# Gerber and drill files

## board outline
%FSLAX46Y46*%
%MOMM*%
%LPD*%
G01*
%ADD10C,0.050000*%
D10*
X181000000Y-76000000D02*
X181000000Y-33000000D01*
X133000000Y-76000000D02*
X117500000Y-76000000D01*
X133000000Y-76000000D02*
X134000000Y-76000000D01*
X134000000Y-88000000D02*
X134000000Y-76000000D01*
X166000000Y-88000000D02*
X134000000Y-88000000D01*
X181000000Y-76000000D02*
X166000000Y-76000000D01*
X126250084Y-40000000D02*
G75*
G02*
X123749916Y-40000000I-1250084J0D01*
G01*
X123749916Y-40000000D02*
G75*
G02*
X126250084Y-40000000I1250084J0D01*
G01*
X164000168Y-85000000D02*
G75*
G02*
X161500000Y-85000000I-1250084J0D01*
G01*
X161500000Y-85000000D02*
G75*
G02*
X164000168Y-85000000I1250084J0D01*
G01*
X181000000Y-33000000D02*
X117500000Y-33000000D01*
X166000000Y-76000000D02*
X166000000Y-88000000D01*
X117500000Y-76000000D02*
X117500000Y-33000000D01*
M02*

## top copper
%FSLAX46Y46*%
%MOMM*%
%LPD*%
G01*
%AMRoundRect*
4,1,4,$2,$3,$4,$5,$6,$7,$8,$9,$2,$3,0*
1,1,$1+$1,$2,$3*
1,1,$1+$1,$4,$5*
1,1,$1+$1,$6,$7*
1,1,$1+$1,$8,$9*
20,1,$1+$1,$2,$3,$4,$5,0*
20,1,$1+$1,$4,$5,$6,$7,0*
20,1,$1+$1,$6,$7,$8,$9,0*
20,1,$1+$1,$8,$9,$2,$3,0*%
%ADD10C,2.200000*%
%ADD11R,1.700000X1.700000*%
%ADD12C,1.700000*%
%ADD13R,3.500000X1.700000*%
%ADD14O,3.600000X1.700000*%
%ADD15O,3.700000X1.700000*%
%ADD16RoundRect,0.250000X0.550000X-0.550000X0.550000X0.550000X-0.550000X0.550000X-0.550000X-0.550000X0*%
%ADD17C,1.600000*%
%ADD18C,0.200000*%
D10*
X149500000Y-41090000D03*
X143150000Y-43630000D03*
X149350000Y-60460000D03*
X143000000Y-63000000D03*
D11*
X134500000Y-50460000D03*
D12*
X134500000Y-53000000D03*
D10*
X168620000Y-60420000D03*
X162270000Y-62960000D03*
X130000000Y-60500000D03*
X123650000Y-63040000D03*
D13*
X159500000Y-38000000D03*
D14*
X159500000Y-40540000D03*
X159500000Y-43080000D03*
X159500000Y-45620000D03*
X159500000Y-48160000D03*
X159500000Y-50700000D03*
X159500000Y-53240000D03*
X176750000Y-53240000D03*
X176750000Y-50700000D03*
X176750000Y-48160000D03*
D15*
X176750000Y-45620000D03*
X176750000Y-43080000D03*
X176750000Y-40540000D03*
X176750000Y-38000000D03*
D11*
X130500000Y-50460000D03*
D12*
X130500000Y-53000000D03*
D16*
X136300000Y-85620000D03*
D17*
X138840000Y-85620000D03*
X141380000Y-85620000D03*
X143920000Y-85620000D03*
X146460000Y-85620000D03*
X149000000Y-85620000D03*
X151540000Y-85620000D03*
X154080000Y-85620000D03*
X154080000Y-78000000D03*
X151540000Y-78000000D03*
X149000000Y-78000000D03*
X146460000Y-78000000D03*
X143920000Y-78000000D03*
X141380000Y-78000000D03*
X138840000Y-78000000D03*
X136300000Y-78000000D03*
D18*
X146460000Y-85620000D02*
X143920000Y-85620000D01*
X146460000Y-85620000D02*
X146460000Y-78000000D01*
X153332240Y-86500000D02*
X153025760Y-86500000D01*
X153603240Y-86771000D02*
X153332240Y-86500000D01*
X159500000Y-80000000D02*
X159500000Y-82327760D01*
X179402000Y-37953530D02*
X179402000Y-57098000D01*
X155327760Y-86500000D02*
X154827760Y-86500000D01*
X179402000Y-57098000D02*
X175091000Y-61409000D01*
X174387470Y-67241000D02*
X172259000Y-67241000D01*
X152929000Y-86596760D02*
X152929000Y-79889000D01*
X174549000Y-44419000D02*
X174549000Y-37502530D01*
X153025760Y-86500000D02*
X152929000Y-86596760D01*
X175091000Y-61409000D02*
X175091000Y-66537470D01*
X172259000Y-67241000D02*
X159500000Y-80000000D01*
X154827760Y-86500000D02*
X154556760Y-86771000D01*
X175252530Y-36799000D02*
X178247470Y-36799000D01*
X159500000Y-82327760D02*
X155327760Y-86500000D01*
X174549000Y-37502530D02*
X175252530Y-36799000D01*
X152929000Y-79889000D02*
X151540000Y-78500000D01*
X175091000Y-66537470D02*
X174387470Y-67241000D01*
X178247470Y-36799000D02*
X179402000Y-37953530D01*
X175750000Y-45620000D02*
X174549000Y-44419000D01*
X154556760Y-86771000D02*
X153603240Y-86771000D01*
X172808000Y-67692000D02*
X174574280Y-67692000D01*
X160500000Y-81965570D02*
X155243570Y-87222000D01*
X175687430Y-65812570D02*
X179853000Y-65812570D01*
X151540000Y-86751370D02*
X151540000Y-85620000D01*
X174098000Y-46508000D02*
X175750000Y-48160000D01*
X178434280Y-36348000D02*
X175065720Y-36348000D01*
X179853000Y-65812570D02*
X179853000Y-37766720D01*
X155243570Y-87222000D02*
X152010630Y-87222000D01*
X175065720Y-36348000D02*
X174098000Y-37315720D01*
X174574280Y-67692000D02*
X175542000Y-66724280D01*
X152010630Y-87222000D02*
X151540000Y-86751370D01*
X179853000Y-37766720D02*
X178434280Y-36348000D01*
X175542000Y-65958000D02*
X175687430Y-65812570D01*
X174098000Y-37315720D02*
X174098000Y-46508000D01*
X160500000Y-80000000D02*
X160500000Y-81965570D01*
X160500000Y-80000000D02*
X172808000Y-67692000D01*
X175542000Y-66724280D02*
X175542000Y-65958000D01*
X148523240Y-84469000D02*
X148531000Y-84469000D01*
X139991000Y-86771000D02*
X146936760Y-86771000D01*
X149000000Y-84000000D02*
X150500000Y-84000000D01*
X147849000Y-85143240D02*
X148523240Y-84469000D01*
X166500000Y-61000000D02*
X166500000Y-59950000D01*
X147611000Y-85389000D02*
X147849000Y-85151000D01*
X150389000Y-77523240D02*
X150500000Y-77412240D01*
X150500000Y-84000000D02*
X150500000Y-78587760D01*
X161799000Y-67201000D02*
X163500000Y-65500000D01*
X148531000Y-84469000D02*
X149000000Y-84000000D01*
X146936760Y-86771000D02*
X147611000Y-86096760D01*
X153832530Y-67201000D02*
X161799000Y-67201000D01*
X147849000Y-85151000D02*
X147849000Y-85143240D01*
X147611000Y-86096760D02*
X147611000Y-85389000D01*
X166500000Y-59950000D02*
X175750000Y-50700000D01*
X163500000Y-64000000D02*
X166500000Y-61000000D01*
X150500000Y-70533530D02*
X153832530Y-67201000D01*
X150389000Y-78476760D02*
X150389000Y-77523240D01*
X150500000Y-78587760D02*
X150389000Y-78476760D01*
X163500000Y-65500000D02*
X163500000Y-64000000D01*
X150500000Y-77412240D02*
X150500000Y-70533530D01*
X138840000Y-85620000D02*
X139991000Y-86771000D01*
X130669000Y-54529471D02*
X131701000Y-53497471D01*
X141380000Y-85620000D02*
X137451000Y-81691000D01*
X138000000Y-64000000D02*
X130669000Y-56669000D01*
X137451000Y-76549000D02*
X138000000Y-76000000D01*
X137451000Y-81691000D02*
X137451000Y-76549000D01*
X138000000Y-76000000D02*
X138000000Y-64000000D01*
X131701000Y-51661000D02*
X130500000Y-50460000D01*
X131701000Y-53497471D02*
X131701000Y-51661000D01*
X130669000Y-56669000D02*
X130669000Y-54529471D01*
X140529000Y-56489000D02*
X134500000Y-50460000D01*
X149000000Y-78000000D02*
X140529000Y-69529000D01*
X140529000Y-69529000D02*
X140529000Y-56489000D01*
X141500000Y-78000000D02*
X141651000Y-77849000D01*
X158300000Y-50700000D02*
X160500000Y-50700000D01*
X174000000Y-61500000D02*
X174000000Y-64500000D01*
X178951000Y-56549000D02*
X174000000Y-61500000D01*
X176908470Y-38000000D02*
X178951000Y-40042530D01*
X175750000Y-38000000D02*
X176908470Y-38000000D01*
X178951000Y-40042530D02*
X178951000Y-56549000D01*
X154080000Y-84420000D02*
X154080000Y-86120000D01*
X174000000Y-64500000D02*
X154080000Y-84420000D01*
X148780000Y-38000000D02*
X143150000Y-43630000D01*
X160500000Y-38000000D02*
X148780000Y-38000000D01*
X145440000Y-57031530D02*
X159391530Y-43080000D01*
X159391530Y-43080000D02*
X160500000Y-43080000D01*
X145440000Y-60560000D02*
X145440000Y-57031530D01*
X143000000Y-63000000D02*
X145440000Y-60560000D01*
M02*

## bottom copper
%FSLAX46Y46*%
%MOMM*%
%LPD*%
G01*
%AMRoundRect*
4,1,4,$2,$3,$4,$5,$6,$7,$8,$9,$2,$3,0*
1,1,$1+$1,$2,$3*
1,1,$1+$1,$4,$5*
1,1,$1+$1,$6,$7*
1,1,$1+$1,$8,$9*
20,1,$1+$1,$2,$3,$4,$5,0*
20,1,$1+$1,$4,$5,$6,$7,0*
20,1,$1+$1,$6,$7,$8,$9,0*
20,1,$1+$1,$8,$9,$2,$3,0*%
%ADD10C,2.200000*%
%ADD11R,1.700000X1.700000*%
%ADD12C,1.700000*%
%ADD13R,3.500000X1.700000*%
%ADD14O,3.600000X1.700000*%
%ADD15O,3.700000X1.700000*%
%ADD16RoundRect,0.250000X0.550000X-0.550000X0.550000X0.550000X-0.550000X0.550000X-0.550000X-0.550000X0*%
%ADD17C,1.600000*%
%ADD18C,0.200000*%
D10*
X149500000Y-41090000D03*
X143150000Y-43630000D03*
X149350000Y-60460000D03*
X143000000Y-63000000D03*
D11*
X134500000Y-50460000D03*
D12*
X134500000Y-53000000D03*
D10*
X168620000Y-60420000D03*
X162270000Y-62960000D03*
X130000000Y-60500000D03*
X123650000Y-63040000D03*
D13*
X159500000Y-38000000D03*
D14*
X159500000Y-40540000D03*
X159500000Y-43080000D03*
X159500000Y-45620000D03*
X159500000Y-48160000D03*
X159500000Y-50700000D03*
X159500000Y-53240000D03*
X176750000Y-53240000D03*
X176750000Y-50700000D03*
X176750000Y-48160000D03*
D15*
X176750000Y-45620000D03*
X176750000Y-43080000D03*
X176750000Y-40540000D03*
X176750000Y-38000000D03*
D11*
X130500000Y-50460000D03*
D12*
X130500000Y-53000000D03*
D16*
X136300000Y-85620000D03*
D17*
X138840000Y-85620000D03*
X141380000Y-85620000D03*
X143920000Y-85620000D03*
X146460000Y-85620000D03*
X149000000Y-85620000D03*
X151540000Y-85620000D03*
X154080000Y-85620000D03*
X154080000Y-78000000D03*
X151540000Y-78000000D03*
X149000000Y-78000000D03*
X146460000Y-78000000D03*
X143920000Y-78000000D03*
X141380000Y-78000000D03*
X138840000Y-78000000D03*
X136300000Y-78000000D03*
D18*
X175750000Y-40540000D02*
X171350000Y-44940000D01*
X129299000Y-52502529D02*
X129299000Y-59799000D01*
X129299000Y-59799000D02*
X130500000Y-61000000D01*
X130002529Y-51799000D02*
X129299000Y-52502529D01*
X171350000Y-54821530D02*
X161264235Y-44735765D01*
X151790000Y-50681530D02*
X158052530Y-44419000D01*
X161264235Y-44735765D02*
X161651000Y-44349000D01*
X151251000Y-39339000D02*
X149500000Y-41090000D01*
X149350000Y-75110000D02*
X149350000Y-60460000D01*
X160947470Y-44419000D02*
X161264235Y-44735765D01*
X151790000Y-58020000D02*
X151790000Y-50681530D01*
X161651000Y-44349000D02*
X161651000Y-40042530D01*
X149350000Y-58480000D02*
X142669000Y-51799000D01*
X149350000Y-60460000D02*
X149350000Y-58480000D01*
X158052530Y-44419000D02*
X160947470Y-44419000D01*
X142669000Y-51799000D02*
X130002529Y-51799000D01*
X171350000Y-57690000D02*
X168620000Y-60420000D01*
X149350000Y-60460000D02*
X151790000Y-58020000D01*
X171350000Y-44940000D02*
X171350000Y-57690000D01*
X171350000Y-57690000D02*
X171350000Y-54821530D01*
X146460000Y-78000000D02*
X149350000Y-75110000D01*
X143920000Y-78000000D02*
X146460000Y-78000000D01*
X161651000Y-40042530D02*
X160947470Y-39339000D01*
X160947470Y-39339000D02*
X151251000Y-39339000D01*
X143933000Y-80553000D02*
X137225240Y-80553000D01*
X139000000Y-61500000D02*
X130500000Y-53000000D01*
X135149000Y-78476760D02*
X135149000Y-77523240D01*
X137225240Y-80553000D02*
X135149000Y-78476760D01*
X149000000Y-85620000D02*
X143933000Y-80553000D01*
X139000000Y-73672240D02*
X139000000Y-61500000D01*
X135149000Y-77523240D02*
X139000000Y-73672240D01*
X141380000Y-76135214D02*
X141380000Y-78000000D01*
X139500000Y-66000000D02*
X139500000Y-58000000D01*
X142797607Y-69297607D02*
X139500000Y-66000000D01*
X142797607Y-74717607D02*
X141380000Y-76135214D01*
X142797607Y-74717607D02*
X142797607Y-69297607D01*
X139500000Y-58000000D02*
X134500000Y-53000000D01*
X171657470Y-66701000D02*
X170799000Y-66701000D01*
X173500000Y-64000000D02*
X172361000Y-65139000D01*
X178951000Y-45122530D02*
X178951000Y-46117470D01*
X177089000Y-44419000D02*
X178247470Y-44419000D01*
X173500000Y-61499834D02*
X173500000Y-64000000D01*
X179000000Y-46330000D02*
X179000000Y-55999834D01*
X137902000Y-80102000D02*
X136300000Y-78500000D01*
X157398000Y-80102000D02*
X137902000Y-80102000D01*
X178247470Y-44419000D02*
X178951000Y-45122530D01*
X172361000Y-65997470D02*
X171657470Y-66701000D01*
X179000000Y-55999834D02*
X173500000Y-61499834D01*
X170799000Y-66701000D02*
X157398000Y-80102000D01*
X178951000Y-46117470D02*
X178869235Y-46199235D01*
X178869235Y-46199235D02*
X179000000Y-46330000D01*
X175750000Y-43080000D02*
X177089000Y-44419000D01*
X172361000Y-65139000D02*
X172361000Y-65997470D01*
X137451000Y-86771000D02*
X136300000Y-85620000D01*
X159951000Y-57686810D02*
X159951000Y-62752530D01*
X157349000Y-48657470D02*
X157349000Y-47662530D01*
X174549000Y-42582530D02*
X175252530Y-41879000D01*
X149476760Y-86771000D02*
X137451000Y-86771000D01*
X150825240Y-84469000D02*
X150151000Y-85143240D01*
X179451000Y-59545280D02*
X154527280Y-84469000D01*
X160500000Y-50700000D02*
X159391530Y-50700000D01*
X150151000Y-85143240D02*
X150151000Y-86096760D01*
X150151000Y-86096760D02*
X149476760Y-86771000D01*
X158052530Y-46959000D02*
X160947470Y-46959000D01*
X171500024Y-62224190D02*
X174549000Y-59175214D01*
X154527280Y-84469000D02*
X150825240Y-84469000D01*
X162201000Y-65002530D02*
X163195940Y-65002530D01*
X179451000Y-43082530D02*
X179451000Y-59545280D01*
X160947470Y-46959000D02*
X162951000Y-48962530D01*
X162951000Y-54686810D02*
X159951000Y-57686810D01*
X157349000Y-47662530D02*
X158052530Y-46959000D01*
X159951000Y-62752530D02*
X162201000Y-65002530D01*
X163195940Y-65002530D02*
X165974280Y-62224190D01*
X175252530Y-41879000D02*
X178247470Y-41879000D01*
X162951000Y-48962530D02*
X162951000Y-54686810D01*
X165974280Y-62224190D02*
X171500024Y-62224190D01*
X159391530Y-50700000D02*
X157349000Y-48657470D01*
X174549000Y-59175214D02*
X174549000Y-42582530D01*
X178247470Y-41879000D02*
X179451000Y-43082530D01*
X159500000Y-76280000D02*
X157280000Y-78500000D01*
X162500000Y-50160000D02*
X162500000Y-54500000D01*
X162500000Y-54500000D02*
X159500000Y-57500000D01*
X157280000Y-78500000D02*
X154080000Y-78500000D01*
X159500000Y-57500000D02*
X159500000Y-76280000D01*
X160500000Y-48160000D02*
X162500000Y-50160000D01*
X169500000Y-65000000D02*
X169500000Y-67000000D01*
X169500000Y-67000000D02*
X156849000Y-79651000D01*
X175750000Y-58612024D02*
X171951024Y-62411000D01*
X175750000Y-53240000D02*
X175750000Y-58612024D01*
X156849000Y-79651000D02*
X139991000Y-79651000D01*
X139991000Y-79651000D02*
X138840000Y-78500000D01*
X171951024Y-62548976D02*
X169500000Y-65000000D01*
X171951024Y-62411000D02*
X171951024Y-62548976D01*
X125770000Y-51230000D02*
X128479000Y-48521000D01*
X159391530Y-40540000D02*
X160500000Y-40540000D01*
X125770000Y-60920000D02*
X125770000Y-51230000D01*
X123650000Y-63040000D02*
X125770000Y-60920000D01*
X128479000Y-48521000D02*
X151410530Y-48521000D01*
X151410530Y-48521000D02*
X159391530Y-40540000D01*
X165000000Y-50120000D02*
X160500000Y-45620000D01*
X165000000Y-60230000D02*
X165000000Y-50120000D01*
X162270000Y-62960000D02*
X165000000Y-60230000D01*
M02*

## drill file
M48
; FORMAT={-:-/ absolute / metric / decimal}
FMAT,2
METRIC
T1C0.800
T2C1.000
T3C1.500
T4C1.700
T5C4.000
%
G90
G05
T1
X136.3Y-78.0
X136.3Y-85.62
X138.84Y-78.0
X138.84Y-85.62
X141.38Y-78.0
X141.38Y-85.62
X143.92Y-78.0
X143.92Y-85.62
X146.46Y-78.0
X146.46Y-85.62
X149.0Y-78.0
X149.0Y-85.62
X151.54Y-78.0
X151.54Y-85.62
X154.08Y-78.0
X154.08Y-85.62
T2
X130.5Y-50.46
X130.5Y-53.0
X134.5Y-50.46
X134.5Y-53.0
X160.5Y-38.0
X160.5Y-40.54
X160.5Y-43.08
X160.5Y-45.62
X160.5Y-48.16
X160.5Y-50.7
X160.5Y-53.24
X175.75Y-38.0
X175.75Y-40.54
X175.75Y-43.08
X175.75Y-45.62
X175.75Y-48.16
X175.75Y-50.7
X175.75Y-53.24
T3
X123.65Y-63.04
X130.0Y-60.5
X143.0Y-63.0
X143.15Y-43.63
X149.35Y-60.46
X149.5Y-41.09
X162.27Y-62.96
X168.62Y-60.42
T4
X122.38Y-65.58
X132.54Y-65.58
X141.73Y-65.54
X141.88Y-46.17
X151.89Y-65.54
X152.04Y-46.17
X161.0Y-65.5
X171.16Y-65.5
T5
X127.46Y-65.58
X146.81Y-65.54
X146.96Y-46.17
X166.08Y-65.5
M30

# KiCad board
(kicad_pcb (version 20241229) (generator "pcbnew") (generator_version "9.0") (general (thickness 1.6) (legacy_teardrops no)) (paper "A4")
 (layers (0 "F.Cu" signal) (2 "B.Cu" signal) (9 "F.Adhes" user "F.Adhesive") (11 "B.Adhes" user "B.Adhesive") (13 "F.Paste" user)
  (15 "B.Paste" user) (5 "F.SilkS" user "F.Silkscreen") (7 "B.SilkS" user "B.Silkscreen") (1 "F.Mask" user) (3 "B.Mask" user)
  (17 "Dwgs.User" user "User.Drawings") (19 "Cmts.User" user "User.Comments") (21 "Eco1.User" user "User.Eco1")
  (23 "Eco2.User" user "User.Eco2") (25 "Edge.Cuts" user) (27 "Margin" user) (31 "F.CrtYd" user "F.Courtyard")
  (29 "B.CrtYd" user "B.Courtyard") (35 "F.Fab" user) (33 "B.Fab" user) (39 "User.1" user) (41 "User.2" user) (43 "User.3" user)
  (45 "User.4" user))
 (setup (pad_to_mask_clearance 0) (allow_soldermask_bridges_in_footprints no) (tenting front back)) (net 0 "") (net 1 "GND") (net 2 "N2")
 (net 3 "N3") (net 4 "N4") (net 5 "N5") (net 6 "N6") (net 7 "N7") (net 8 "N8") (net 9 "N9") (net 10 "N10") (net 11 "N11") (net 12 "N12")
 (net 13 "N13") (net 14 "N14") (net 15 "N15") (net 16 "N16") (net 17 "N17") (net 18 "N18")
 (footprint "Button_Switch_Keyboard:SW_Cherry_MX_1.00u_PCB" (layer "F.Cu") (at 149.5 41.09)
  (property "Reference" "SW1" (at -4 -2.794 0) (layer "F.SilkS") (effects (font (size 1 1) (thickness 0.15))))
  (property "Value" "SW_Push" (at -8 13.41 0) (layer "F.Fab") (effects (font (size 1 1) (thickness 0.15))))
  (pad "" np_thru_hole circle (at -7.62 5.08) (size 1.7 1.7) (drill 1.7) (layers "*.Cu" "*.Mask"))
  (pad "" np_thru_hole circle (at -2.54 5.08) (size 4 4) (drill 4) (layers "*.Cu" "*.Mask"))
  (pad "" np_thru_hole circle (at 2.54 5.08) (size 1.7 1.7) (drill 1.7) (layers "*.Cu" "*.Mask"))
  (pad "1" thru_hole circle (at 0 0) (size 2.2 2.2) (drill 1.5) (layers "*.Cu" "*.Mask") (remove_unused_layers no) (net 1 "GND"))
  (pad "2" thru_hole circle (at -6.35 2.54) (size 2.2 2.2) (drill 1.5) (layers "*.Cu" "*.Mask") (remove_unused_layers no) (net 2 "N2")))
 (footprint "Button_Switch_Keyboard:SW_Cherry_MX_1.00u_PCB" (layer "F.Cu") (at 149.35 60.46)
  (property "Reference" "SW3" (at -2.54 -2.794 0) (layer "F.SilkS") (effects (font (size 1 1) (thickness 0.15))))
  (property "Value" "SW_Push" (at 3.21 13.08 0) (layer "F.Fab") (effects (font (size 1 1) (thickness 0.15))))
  (pad "" np_thru_hole circle (at -7.62 5.08) (size 1.7 1.7) (drill 1.7) (layers "*.Cu" "*.Mask"))
  (pad "" np_thru_hole circle (at -2.54 5.08) (size 4 4) (drill 4) (layers "*.Cu" "*.Mask"))
  (pad "" np_thru_hole circle (at 2.54 5.08) (size 1.7 1.7) (drill 1.7) (layers "*.Cu" "*.Mask"))
  (pad "1" thru_hole circle (at 0 0) (size 2.2 2.2) (drill 1.5) (layers "*.Cu" "*.Mask") (remove_unused_layers no) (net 1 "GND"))
  (pad "2" thru_hole circle (at -6.35 2.54) (size 2.2 2.2) (drill 1.5) (layers "*.Cu" "*.Mask") (remove_unused_layers no) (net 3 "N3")))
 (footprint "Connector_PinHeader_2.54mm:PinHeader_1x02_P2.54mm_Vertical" (layer "F.Cu") (at 134.5 50.46)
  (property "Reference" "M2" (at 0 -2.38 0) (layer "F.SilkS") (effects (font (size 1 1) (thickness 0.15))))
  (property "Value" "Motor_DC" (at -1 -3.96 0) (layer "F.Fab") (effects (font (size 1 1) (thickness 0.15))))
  (pad "1" thru_hole rect (at 0 0) (size 1.7 1.7) (drill 1) (layers "*.Cu" "*.Mask") (remove_unused_layers no) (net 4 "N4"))
  (pad "2" thru_hole circle (at 0 2.54) (size 1.7 1.7) (drill 1) (layers "*.Cu" "*.Mask") (remove_unused_layers no) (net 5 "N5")))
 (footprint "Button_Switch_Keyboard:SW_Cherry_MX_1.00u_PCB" (layer "F.Cu") (at 168.62 60.42)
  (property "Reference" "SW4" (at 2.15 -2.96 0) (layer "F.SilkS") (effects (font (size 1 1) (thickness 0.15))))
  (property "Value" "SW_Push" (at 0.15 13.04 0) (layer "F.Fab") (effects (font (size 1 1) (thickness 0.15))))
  (pad "" np_thru_hole circle (at -7.62 5.08) (size 1.7 1.7) (drill 1.7) (layers "*.Cu" "*.Mask"))
  (pad "" np_thru_hole circle (at -2.54 5.08) (size 4 4) (drill 4) (layers "*.Cu" "*.Mask"))
  (pad "" np_thru_hole circle (at 2.54 5.08) (size 1.7 1.7) (drill 1.7) (layers "*.Cu" "*.Mask"))
  (pad "1" thru_hole circle (at 0 0) (size 2.2 2.2) (drill 1.5) (layers "*.Cu" "*.Mask") (remove_unused_layers no) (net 1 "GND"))
  (pad "2" thru_hole circle (at -6.35 2.54) (size 2.2 2.2) (drill 1.5) (layers "*.Cu" "*.Mask") (remove_unused_layers no) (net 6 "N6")))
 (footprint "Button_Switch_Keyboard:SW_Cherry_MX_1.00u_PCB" (layer "F.Cu") (at 130 60.5)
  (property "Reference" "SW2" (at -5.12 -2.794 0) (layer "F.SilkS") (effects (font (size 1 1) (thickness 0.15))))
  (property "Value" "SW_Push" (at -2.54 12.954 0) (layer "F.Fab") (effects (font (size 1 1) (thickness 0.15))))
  (pad "" np_thru_hole circle (at -7.62 5.08) (size 1.7 1.7) (drill 1.7) (layers "*.Cu" "*.Mask"))
  (pad "" np_thru_hole circle (at -2.54 5.08) (size 4 4) (drill 4) (layers "*.Cu" "*.Mask"))
  (pad "" np_thru_hole circle (at 2.54 5.08) (size 1.7 1.7) (drill 1.7) (layers "*.Cu" "*.Mask"))
  (pad "1" thru_hole circle (at 0 0) (size 2.2 2.2) (drill 1.5) (layers "*.Cu" "*.Mask") (remove_unused_layers no) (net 1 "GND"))
  (pad "2" thru_hole circle (at -6.35 2.54) (size 2.2 2.2) (drill 1.5) (layers "*.Cu" "*.Mask") (remove_unused_layers no) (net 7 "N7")))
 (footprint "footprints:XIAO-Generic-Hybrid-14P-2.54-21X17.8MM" (layer "F.Cu") (at 168.125 45.62)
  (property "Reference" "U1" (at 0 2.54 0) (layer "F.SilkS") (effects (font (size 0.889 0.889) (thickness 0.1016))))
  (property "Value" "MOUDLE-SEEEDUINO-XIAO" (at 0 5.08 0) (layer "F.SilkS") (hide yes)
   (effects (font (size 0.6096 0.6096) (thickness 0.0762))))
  (pad "1" thru_hole rect (at -7.625 -7.62) (size 3.5 1.7) (drill 1 (offset -1 0)) (layers "*.Cu" "*.Mask") (remove_unused_layers no)
   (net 2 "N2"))
  (pad "2" thru_hole oval (at -7.625 -5.08) (size 3.6 1.7) (drill 1 (offset -1 0)) (layers "*.Cu" "*.Mask") (remove_unused_layers no)
   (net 7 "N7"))
  (pad "3" thru_hole oval (at -7.625 -2.54) (size 3.6 1.7) (drill 1 (offset -1 0)) (layers "*.Cu" "*.Mask") (remove_unused_layers no)
   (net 3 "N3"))
  (pad "4" thru_hole oval (at -7.625 0) (size 3.6 1.7) (drill 1 (offset -1 0)) (layers "*.Cu" "*.Mask") (remove_unused_layers no)
   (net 6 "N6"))
  (pad "5" thru_hole oval (at -7.625 2.54) (size 3.6 1.7) (drill 1 (offset -1 0)) (layers "*.Cu" "*.Mask") (remove_unused_layers no)
   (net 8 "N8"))
  (pad "6" thru_hole oval (at -7.625 5.08 180) (size 3.6 1.7) (drill 1 (offset 1 0)) (layers "*.Cu" "*.Mask") (remove_unused_layers no)
   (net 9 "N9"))
  (pad "7" thru_hole oval (at -7.625 7.62) (size 3.6 1.7) (drill 1 (offset -1 0)) (layers "*.Cu" "*.Mask") (remove_unused_layers no)
   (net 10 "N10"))
  (pad "8" thru_hole oval (at 7.625 7.62) (size 3.6 1.7) (drill 1 (offset 1 0)) (layers "*.Cu" "*.Mask") (remove_unused_layers no)
   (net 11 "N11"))
  (pad "9" thru_hole oval (at 7.625 5.08) (size 3.6 1.7) (drill 1 (offset 1 0)) (layers "*.Cu" "*.Mask") (remove_unused_layers no)
   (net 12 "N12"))
  (pad "10" thru_hole oval (at 7.625 2.54) (size 3.6 1.7) (drill 1 (offset 1 0)) (layers "*.Cu" "*.Mask") (remove_unused_layers no)
   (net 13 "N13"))
  (pad "11" thru_hole oval (at 7.625 0) (size 3.7 1.7) (drill 1 (offset 1 0)) (layers "*.Cu" "*.Mask") (remove_unused_layers no)
   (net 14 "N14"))
  (pad "12" thru_hole oval (at 7.625 -2.54) (size 3.7 1.7) (drill 1 (offset 1 0)) (layers "*.Cu" "*.Mask") (remove_unused_layers no)
   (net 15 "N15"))
  (pad "13" thru_hole oval (at 7.625 -5.08) (size 3.7 1.7) (drill 1 (offset 1 0)) (layers "*.Cu" "*.Mask") (remove_unused_layers no)
   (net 1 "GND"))
  (pad "14" thru_hole oval (at 7.625 -7.62) (size 3.7 1.7) (drill 1 (offset 1 0)) (layers "*.Cu" "*.Mask") (remove_unused_layers no)
   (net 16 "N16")))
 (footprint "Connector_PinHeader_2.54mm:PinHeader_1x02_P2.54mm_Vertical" (layer "F.Cu") (at 130.5 50.46)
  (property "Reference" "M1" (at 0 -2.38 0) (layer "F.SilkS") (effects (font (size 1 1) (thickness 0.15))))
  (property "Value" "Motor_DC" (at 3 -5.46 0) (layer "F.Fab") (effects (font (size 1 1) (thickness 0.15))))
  (pad "1" thru_hole rect (at 0 0) (size 1.7 1.7) (drill 1) (layers "*.Cu" "*.Mask") (remove_unused_layers no) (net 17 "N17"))
  (pad "2" thru_hole circle (at 0 2.54) (size 1.7 1.7) (drill 1) (layers "*.Cu" "*.Mask") (remove_unused_layers no) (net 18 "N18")))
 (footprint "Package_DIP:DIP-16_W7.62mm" (layer "F.Cu") (at 136.3 85.62 90)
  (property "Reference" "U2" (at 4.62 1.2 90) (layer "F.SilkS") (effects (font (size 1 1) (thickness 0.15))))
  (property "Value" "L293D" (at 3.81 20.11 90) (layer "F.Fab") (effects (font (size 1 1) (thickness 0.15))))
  (pad "1" thru_hole roundrect (at 0 0 90) (size 1.6 1.6) (drill 0.8) (layers "*.Cu" "*.Mask") (remove_unused_layers no)
   (roundrect_rratio 0.15625) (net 9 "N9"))
  (pad "2" thru_hole circle (at 0 2.54 90) (size 1.6 1.6) (drill 0.8) (layers "*.Cu" "*.Mask") (remove_unused_layers no) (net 12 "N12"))
  (pad "3" thru_hole circle (at 0 5.08 90) (size 1.6 1.6) (drill 0.8) (layers "*.Cu" "*.Mask") (remove_unused_layers no) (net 17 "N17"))
  (pad "4" thru_hole circle (at 0 7.62 90) (size 1.6 1.6) (drill 0.8) (layers "*.Cu" "*.Mask") (remove_unused_layers no) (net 1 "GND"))
  (pad "5" thru_hole circle (at 0 10.16 90) (size 1.6 1.6) (drill 0.8) (layers "*.Cu" "*.Mask") (remove_unused_layers no) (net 1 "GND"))
  (pad "6" thru_hole circle (at 0 12.7 90) (size 1.6 1.6) (drill 0.8) (layers "*.Cu" "*.Mask") (remove_unused_layers no) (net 18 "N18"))
  (pad "7" thru_hole circle (at 0 15.24 90) (size 1.6 1.6) (drill 0.8) (layers "*.Cu" "*.Mask") (remove_unused_layers no) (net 13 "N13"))
  (pad "8" thru_hole circle (at 0 17.78 90) (size 1.6 1.6) (drill 0.8) (layers "*.Cu" "*.Mask") (remove_unused_layers no) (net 16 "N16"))
  (pad "9" thru_hole circle (at 7.62 17.78 90) (size 1.6 1.6) (drill 0.8) (layers "*.Cu" "*.Mask") (remove_unused_layers no) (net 8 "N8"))
  (pad "10" thru_hole circle (at 7.62 15.24 90) (size 1.6 1.6) (drill 0.8) (layers "*.Cu" "*.Mask") (remove_unused_layers no) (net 14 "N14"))
  (pad "11" thru_hole circle (at 7.62 12.7 90) (size 1.6 1.6) (drill 0.8) (layers "*.Cu" "*.Mask") (remove_unused_layers no) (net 4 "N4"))
  (pad "12" thru_hole circle (at 7.62 10.16 90) (size 1.6 1.6) (drill 0.8) (layers "*.Cu" "*.Mask") (remove_unused_layers no) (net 1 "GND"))
  (pad "13" thru_hole circle (at 7.62 7.62 90) (size 1.6 1.6) (drill 0.8) (layers "*.Cu" "*.Mask") (remove_unused_layers no) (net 1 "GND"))
  (pad "14" thru_hole circle (at 7.62 5.08 90) (size 1.6 1.6) (drill 0.8) (layers "*.Cu" "*.Mask") (remove_unused_layers no) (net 5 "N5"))
  (pad "15" thru_hole circle (at 7.62 2.54 90) (size 1.6 1.6) (drill 0.8) (layers "*.Cu" "*.Mask") (remove_unused_layers no) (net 11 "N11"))
  (pad "16" thru_hole circle (at 7.62 0 90) (size 1.6 1.6) (drill 0.8) (layers "*.Cu" "*.Mask") (remove_unused_layers no) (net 15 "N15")))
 (gr_line (start 181 76) (end 181 33) (stroke (width 0.05) (type default)) (layer "Edge.Cuts"))
 (gr_line (start 133 76) (end 117.5 76) (stroke (width 0.05) (type default)) (layer "Edge.Cuts"))
 (gr_line (start 133 76) (end 134 76) (stroke (width 0.05) (type default)) (layer "Edge.Cuts"))
 (gr_line (start 134 88) (end 134 76) (stroke (width 0.05) (type default)) (layer "Edge.Cuts"))
 (gr_line (start 166 88) (end 134 88) (stroke (width 0.05) (type default)) (layer "Edge.Cuts"))
 (gr_line (start 181 76) (end 166 76) (stroke (width 0.05) (type default)) (layer "Edge.Cuts"))
 (gr_circle (center 125 40) (end 123.749916 40) (stroke (width 0.05) (type default)) (fill no) (layer "Edge.Cuts"))
 (gr_circle (center 162.750084 85) (end 161.5 85) (stroke (width 0.05) (type default)) (fill no) (layer "Edge.Cuts"))
 (gr_line (start 181 33) (end 117.5 33) (stroke (width 0.05) (type default)) (layer "Edge.Cuts"))
 (gr_line (start 166 76) (end 166 88) (stroke (width 0.05) (type default)) (layer "Edge.Cuts"))
 (gr_line (start 117.5 76) (end 117.5 33) (stroke (width 0.05) (type default)) (layer "Edge.Cuts"))
 (segment (start 146.46 85.62) (end 143.92 85.62) (width 0.2) (layer "F.Cu") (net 1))
 (segment (start 146.46 85.62) (end 146.46 78) (width 0.2) (layer "F.Cu") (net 1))
 (segment (start 175.75 40.54) (end 171.35 44.94) (width 0.2) (layer "B.Cu") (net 1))
 (segment (start 129.299 52.502529) (end 129.299 59.799) (width 0.2) (layer "B.Cu") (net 1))
 (segment (start 129.299 59.799) (end 130.5 61) (width 0.2) (layer "B.Cu") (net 1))
 (segment (start 130.002529 51.799) (end 129.299 52.502529) (width 0.2) (layer "B.Cu") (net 1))
 (segment (start 171.35 54.82153) (end 161.264235 44.735765) (width 0.2) (layer "B.Cu") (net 1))
 (segment (start 151.79 50.68153) (end 158.05253 44.419) (width 0.2) (layer "B.Cu") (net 1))
 (segment (start 161.264235 44.735765) (end 161.651 44.349) (width 0.2) (layer "B.Cu") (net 1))
 (segment (start 151.251 39.339) (end 149.5 41.09) (width 0.2) (layer "B.Cu") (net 1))
 (segment (start 149.35 75.11) (end 149.35 60.46) (width 0.2) (layer "B.Cu") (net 1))
 (segment (start 160.94747 44.419) (end 161.264235 44.735765) (width 0.2) (layer "B.Cu") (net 1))
 (segment (start 151.79 58.02) (end 151.79 50.68153) (width 0.2) (layer "B.Cu") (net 1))
 (segment (start 161.651 44.349) (end 161.651 40.04253) (width 0.2) (layer "B.Cu") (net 1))
 (segment (start 149.35 58.48) (end 142.669 51.799) (width 0.2) (layer "B.Cu") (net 1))
 (segment (start 149.35 60.46) (end 149.35 58.48) (width 0.2) (layer "B.Cu") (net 1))
 (segment (start 158.05253 44.419) (end 160.94747 44.419) (width 0.2) (layer "B.Cu") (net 1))
 (segment (start 142.669 51.799) (end 130.002529 51.799) (width 0.2) (layer "B.Cu") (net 1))
 (segment (start 171.35 57.69) (end 168.62 60.42) (width 0.2) (layer "B.Cu") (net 1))
 (segment (start 149.35 60.46) (end 151.79 58.02) (width 0.2) (layer "B.Cu") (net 1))
 (segment (start 171.35 44.94) (end 171.35 57.69) (width 0.2) (layer "B.Cu") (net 1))
 (segment (start 171.35 57.69) (end 171.35 54.82153) (width 0.2) (layer "B.Cu") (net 1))
 (segment (start 146.46 78) (end 149.35 75.11) (width 0.2) (layer "B.Cu") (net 1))
 (segment (start 143.92 78) (end 146.46 78) (width 0.2) (layer "B.Cu") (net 1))
 (segment (start 161.651 40.04253) (end 160.94747 39.339) (width 0.2) (layer "B.Cu") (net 1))
 (segment (start 160.94747 39.339) (end 151.251 39.339) (width 0.2) (layer "B.Cu") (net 1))
 (segment (start 153.33224 86.5) (end 153.02576 86.5) (width 0.2) (layer "F.Cu") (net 14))
 (segment (start 153.60324 86.771) (end 153.33224 86.5) (width 0.2) (layer "F.Cu") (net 14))
 (segment (start 159.5 80) (end 159.5 82.32776) (width 0.2) (layer "F.Cu") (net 14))
 (segment (start 179.402 37.95353) (end 179.402 57.098) (width 0.2) (layer "F.Cu") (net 14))
 (segment (start 155.32776 86.5) (end 154.82776 86.5) (width 0.2) (layer "F.Cu") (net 14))
 (segment (start 179.402 57.098) (end 175.091 61.409) (width 0.2) (layer "F.Cu") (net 14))
 (segment (start 174.38747 67.241) (end 172.259 67.241) (width 0.2) (layer "F.Cu") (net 14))
 (segment (start 152.929 86.59676) (end 152.929 79.889) (width 0.2) (layer "F.Cu") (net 14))
 (segment (start 174.549 44.419) (end 174.549 37.50253) (width 0.2) (layer "F.Cu") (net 14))
 (segment (start 153.02576 86.5) (end 152.929 86.59676) (width 0.2) (layer "F.Cu") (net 14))
 (segment (start 175.091 61.409) (end 175.091 66.53747) (width 0.2) (layer "F.Cu") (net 14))
 (segment (start 172.259 67.241) (end 159.5 80) (width 0.2) (layer "F.Cu") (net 14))
 (segment (start 154.82776 86.5) (end 154.55676 86.771) (width 0.2) (layer "F.Cu") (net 14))
 (segment (start 175.25253 36.799) (end 178.24747 36.799) (width 0.2) (layer "F.Cu") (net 14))
 (segment (start 159.5 82.32776) (end 155.32776 86.5) (width 0.2) (layer "F.Cu") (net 14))
 (segment (start 174.549 37.50253) (end 175.25253 36.799) (width 0.2) (layer "F.Cu") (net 14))
 (segment (start 152.929 79.889) (end 151.54 78.5) (width 0.2) (layer "F.Cu") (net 14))
 (segment (start 175.091 66.53747) (end 174.38747 67.241) (width 0.2) (layer "F.Cu") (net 14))
 (segment (start 178.24747 36.799) (end 179.402 37.95353) (width 0.2) (layer "F.Cu") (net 14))
 (segment (start 175.75 45.62) (end 174.549 44.419) (width 0.2) (layer "F.Cu") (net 14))
 (segment (start 154.55676 86.771) (end 153.60324 86.771) (width 0.2) (layer "F.Cu") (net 14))
 (segment (start 172.808 67.692) (end 174.57428 67.692) (width 0.2) (layer "F.Cu") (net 13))
 (segment (start 160.5 81.96557) (end 155.24357 87.222) (width 0.2) (layer "F.Cu") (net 13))
 (segment (start 175.68743 65.81257) (end 179.853 65.81257) (width 0.2) (layer "F.Cu") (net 13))
 (segment (start 151.54 86.75137) (end 151.54 85.62) (width 0.2) (layer "F.Cu") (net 13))
 (segment (start 174.098 46.508) (end 175.75 48.16) (width 0.2) (layer "F.Cu") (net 13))
 (segment (start 178.43428 36.348) (end 175.06572 36.348) (width 0.2) (layer "F.Cu") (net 13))
 (segment (start 179.853 65.81257) (end 179.853 37.76672) (width 0.2) (layer "F.Cu") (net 13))
 (segment (start 155.24357 87.222) (end 152.01063 87.222) (width 0.2) (layer "F.Cu") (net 13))
 (segment (start 175.06572 36.348) (end 174.098 37.31572) (width 0.2) (layer "F.Cu") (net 13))
 (segment (start 174.57428 67.692) (end 175.542 66.72428) (width 0.2) (layer "F.Cu") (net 13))
 (segment (start 152.01063 87.222) (end 151.54 86.75137) (width 0.2) (layer "F.Cu") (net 13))
 (segment (start 179.853 37.76672) (end 178.43428 36.348) (width 0.2) (layer "F.Cu") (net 13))
 (segment (start 175.542 65.958) (end 175.68743 65.81257) (width 0.2) (layer "F.Cu") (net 13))
 (segment (start 174.098 37.31572) (end 174.098 46.508) (width 0.2) (layer "F.Cu") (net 13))
 (segment (start 160.5 80) (end 160.5 81.96557) (width 0.2) (layer "F.Cu") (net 13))
 (segment (start 160.5 80) (end 172.808 67.692) (width 0.2) (layer "F.Cu") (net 13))
 (segment (start 175.542 66.72428) (end 175.542 65.958) (width 0.2) (layer "F.Cu") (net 13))
 (segment (start 148.52324 84.469) (end 148.531 84.469) (width 0.2) (layer "F.Cu") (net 12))
 (segment (start 139.991 86.771) (end 146.93676 86.771) (width 0.2) (layer "F.Cu") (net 12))
 (segment (start 149 84) (end 150.5 84) (width 0.2) (layer "F.Cu") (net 12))
 (segment (start 147.849 85.14324) (end 148.52324 84.469) (width 0.2) (layer "F.Cu") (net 12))
 (segment (start 166.5 61) (end 166.5 59.95) (width 0.2) (layer "F.Cu") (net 12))
 (segment (start 147.611 85.389) (end 147.849 85.151) (width 0.2) (layer "F.Cu") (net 12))
 (segment (start 150.389 77.52324) (end 150.5 77.41224) (width 0.2) (layer "F.Cu") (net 12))
 (segment (start 150.5 84) (end 150.5 78.58776) (width 0.2) (layer "F.Cu") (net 12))
 (segment (start 161.799 67.201) (end 163.5 65.5) (width 0.2) (layer "F.Cu") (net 12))
 (segment (start 148.531 84.469) (end 149 84) (width 0.2) (layer "F.Cu") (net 12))
 (segment (start 146.93676 86.771) (end 147.611 86.09676) (width 0.2) (layer "F.Cu") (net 12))
 (segment (start 153.83253 67.201) (end 161.799 67.201) (width 0.2) (layer "F.Cu") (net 12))
 (segment (start 147.849 85.151) (end 147.849 85.14324) (width 0.2) (layer "F.Cu") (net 12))
 (segment (start 147.611 86.09676) (end 147.611 85.389) (width 0.2) (layer "F.Cu") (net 12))
 (segment (start 166.5 59.95) (end 175.75 50.7) (width 0.2) (layer "F.Cu") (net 12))
 (segment (start 163.5 64) (end 166.5 61) (width 0.2) (layer "F.Cu") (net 12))
 (segment (start 150.5 70.53353) (end 153.83253 67.201) (width 0.2) (layer "F.Cu") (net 12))
 (segment (start 150.389 78.47676) (end 150.389 77.52324) (width 0.2) (layer "F.Cu") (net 12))
 (segment (start 150.5 78.58776) (end 150.389 78.47676) (width 0.2) (layer "F.Cu") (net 12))
 (segment (start 163.5 65.5) (end 163.5 64) (width 0.2) (layer "F.Cu") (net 12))
 (segment (start 150.5 77.41224) (end 150.5 70.53353) (width 0.2) (layer "F.Cu") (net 12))
 (segment (start 138.84 85.62) (end 139.991 86.771) (width 0.2) (layer "F.Cu") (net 12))
 (segment (start 130.669 54.529471) (end 131.701 53.497471) (width 0.2) (layer "F.Cu") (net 17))
 (segment (start 141.38 85.62) (end 137.451 81.691) (width 0.2) (layer "F.Cu") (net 17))
 (segment (start 138 64) (end 130.669 56.669) (width 0.2) (layer "F.Cu") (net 17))
 (segment (start 137.451 76.549) (end 138 76) (width 0.2) (layer "F.Cu") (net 17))
 (segment (start 137.451 81.691) (end 137.451 76.549) (width 0.2) (layer "F.Cu") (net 17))
 (segment (start 138 76) (end 138 64) (width 0.2) (layer "F.Cu") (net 17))
 (segment (start 131.701 51.661) (end 130.5 50.46) (width 0.2) (layer "F.Cu") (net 17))
 (segment (start 131.701 53.497471) (end 131.701 51.661) (width 0.2) (layer "F.Cu") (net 17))
 (segment (start 130.669 56.669) (end 130.669 54.529471) (width 0.2) (layer "F.Cu") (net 17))
 (segment (start 143.933 80.553) (end 137.22524 80.553) (width 0.2) (layer "B.Cu") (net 18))
 (segment (start 139 61.5) (end 130.5 53) (width 0.2) (layer "B.Cu") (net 18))
 (segment (start 135.149 78.47676) (end 135.149 77.52324) (width 0.2) (layer "B.Cu") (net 18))
 (segment (start 137.22524 80.553) (end 135.149 78.47676) (width 0.2) (layer "B.Cu") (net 18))
 (segment (start 149 85.62) (end 143.933 80.553) (width 0.2) (layer "B.Cu") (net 18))
 (segment (start 139 73.67224) (end 139 61.5) (width 0.2) (layer "B.Cu") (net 18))
 (segment (start 135.149 77.52324) (end 139 73.67224) (width 0.2) (layer "B.Cu") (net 18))
 (segment (start 140.529 56.489) (end 134.5 50.46) (width 0.2) (layer "F.Cu") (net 4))
 (segment (start 149 78) (end 140.529 69.529) (width 0.2) (layer "F.Cu") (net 4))
 (segment (start 140.529 69.529) (end 140.529 56.489) (width 0.2) (layer "F.Cu") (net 4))
 (segment (start 141.5 78) (end 141.651 77.849) (width 0.2) (layer "F.Cu") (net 5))
 (segment (start 141.38 76.135214) (end 141.38 78) (width 0.2) (layer "B.Cu") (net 5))
 (segment (start 139.5 66) (end 139.5 58) (width 0.2) (layer "B.Cu") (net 5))
 (segment (start 142.797607 69.297607) (end 139.5 66) (width 0.2) (layer "B.Cu") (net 5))
 (segment (start 142.797607 74.717607) (end 141.38 76.135214) (width 0.2) (layer "B.Cu") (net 5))
 (segment (start 142.797607 74.717607) (end 142.797607 69.297607) (width 0.2) (layer "B.Cu") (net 5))
 (segment (start 139.5 58) (end 134.5 53) (width 0.2) (layer "B.Cu") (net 5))
 (segment (start 171.65747 66.701) (end 170.799 66.701) (width 0.2) (layer "B.Cu") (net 15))
 (segment (start 173.5 64) (end 172.361 65.139) (width 0.2) (layer "B.Cu") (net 15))
 (segment (start 178.951 45.12253) (end 178.951 46.11747) (width 0.2) (layer "B.Cu") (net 15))
 (segment (start 177.089 44.419) (end 178.24747 44.419) (width 0.2) (layer "B.Cu") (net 15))
 (segment (start 173.5 61.499834) (end 173.5 64) (width 0.2) (layer "B.Cu") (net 15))
 (segment (start 179 46.33) (end 179 55.999834) (width 0.2) (layer "B.Cu") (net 15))
 (segment (start 137.902 80.102) (end 136.3 78.5) (width 0.2) (layer "B.Cu") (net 15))
 (segment (start 157.398 80.102) (end 137.902 80.102) (width 0.2) (layer "B.Cu") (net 15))
 (segment (start 178.24747 44.419) (end 178.951 45.12253) (width 0.2) (layer "B.Cu") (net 15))
 (segment (start 172.361 65.99747) (end 171.65747 66.701) (width 0.2) (layer "B.Cu") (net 15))
 (segment (start 179 55.999834) (end 173.5 61.499834) (width 0.2) (layer "B.Cu") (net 15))
 (segment (start 170.799 66.701) (end 157.398 80.102) (width 0.2) (layer "B.Cu") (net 15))
 (segment (start 178.951 46.11747) (end 178.869235 46.199235) (width 0.2) (layer "B.Cu") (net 15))
 (segment (start 178.869235 46.199235) (end 179 46.33) (width 0.2) (layer "B.Cu") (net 15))
 (segment (start 175.75 43.08) (end 177.089 44.419) (width 0.2) (layer "B.Cu") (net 15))
 (segment (start 172.361 65.139) (end 172.361 65.99747) (width 0.2) (layer "B.Cu") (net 15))
 (segment (start 158.3 50.7) (end 160.5 50.7) (width 0.2) (layer "F.Cu") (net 9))
 (segment (start 137.451 86.771) (end 136.3 85.62) (width 0.2) (layer "B.Cu") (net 9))
 (segment (start 159.951 57.68681) (end 159.951 62.75253) (width 0.2) (layer "B.Cu") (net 9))
 (segment (start 157.349 48.65747) (end 157.349 47.66253) (width 0.2) (layer "B.Cu") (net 9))
 (segment (start 174.549 42.58253) (end 175.25253 41.879) (width 0.2) (layer "B.Cu") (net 9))
 (segment (start 149.47676 86.771) (end 137.451 86.771) (width 0.2) (layer "B.Cu") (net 9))
 (segment (start 150.82524 84.469) (end 150.151 85.14324) (width 0.2) (layer "B.Cu") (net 9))
 (segment (start 179.451 59.54528) (end 154.52728 84.469) (width 0.2) (layer "B.Cu") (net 9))
 (segment (start 160.5 50.7) (end 159.39153 50.7) (width 0.2) (layer "B.Cu") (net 9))
 (segment (start 150.151 85.14324) (end 150.151 86.09676) (width 0.2) (layer "B.Cu") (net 9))
 (segment (start 150.151 86.09676) (end 149.47676 86.771) (width 0.2) (layer "B.Cu") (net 9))
 (segment (start 158.05253 46.959) (end 160.94747 46.959) (width 0.2) (layer "B.Cu") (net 9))
 (segment (start 171.500024 62.22419) (end 174.549 59.175214) (width 0.2) (layer "B.Cu") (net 9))
 (segment (start 154.52728 84.469) (end 150.82524 84.469) (width 0.2) (layer "B.Cu") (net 9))
 (segment (start 162.201 65.00253) (end 163.19594 65.00253) (width 0.2) (layer "B.Cu") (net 9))
 (segment (start 179.451 43.08253) (end 179.451 59.54528) (width 0.2) (layer "B.Cu") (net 9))
 (segment (start 160.94747 46.959) (end 162.951 48.96253) (width 0.2) (layer "B.Cu") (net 9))
 (segment (start 162.951 54.68681) (end 159.951 57.68681) (width 0.2) (layer "B.Cu") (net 9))
 (segment (start 157.349 47.66253) (end 158.05253 46.959) (width 0.2) (layer "B.Cu") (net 9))
 (segment (start 159.951 62.75253) (end 162.201 65.00253) (width 0.2) (layer "B.Cu") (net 9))
 (segment (start 163.19594 65.00253) (end 165.97428 62.22419) (width 0.2) (layer "B.Cu") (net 9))
 (segment (start 175.25253 41.879) (end 178.24747 41.879) (width 0.2) (layer "B.Cu") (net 9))
 (segment (start 162.951 48.96253) (end 162.951 54.68681) (width 0.2) (layer "B.Cu") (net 9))
 (segment (start 165.97428 62.22419) (end 171.500024 62.22419) (width 0.2) (layer "B.Cu") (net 9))
 (segment (start 159.39153 50.7) (end 157.349 48.65747) (width 0.2) (layer "B.Cu") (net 9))
 (segment (start 174.549 59.175214) (end 174.549 42.58253) (width 0.2) (layer "B.Cu") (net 9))
 (segment (start 178.24747 41.879) (end 179.451 43.08253) (width 0.2) (layer "B.Cu") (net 9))
 (segment (start 159.5 76.28) (end 157.28 78.5) (width 0.2) (layer "B.Cu") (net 8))
 (segment (start 162.5 50.16) (end 162.5 54.5) (width 0.2) (layer "B.Cu") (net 8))
 (segment (start 162.5 54.5) (end 159.5 57.5) (width 0.2) (layer "B.Cu") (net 8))
 (segment (start 157.28 78.5) (end 154.08 78.5) (width 0.2) (layer "B.Cu") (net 8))
 (segment (start 159.5 57.5) (end 159.5 76.28) (width 0.2) (layer "B.Cu") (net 8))
 (segment (start 160.5 48.16) (end 162.5 50.16) (width 0.2) (layer "B.Cu") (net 8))
 (segment (start 174 61.5) (end 174 64.5) (width 0.2) (layer "F.Cu") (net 16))
 (segment (start 178.951 56.549) (end 174 61.5) (width 0.2) (layer "F.Cu") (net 16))
 (segment (start 176.90847 38) (end 178.951 40.04253) (width 0.2) (layer "F.Cu") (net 16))
 (segment (start 175.75 38) (end 176.90847 38) (width 0.2) (layer "F.Cu") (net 16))
 (segment (start 178.951 40.04253) (end 178.951 56.549) (width 0.2) (layer "F.Cu") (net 16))
 (segment (start 154.08 84.42) (end 154.08 86.12) (width 0.2) (layer "F.Cu") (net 16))
 (segment (start 174 64.5) (end 154.08 84.42) (width 0.2) (layer "F.Cu") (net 16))
 (segment (start 169.5 65) (end 169.5 67) (width 0.2) (layer "B.Cu") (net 11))
 (segment (start 169.5 67) (end 156.849 79.651) (width 0.2) (layer "B.Cu") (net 11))
 (segment (start 175.75 58.612024) (end 171.951024 62.411) (width 0.2) (layer "B.Cu") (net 11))
 (segment (start 175.75 53.24) (end 175.75 58.612024) (width 0.2) (layer "B.Cu") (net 11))
 (segment (start 156.849 79.651) (end 139.991 79.651) (width 0.2) (layer "B.Cu") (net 11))
 (segment (start 139.991 79.651) (end 138.84 78.5) (width 0.2) (layer "B.Cu") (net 11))
 (segment (start 171.951024 62.548976) (end 169.5 65) (width 0.2) (layer "B.Cu") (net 11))
 (segment (start 171.951024 62.411) (end 171.951024 62.548976) (width 0.2) (layer "B.Cu") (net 11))
 (segment (start 148.78 38) (end 143.15 43.63) (width 0.2) (layer "F.Cu") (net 2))
 (segment (start 160.5 38) (end 148.78 38) (width 0.2) (layer "F.Cu") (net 2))
 (segment (start 125.77 51.23) (end 128.479 48.521) (width 0.2) (layer "B.Cu") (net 7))
 (segment (start 159.39153 40.54) (end 160.5 40.54) (width 0.2) (layer "B.Cu") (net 7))
 (segment (start 125.77 60.92) (end 125.77 51.23) (width 0.2) (layer "B.Cu") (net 7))
 (segment (start 123.65 63.04) (end 125.77 60.92) (width 0.2) (layer "B.Cu") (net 7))
 (segment (start 128.479 48.521) (end 151.41053 48.521) (width 0.2) (layer "B.Cu") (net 7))
 (segment (start 151.41053 48.521) (end 159.39153 40.54) (width 0.2) (layer "B.Cu") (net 7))
 (segment (start 145.44 57.03153) (end 159.39153 43.08) (width 0.2) (layer "F.Cu") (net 3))
 (segment (start 159.39153 43.08) (end 160.5 43.08) (width 0.2) (layer "F.Cu") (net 3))
 (segment (start 145.44 60.56) (end 145.44 57.03153) (width 0.2) (layer "F.Cu") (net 3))
 (segment (start 143 63) (end 145.44 60.56) (width 0.2) (layer "F.Cu") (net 3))
 (segment (start 165 50.12) (end 160.5 45.62) (width 0.2) (layer "B.Cu") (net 6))
 (segment (start 165 60.23) (end 165 50.12) (width 0.2) (layer "B.Cu") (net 6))
 (segment (start 162.27 62.96) (end 165 60.23) (width 0.2) (layer "B.Cu") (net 6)))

